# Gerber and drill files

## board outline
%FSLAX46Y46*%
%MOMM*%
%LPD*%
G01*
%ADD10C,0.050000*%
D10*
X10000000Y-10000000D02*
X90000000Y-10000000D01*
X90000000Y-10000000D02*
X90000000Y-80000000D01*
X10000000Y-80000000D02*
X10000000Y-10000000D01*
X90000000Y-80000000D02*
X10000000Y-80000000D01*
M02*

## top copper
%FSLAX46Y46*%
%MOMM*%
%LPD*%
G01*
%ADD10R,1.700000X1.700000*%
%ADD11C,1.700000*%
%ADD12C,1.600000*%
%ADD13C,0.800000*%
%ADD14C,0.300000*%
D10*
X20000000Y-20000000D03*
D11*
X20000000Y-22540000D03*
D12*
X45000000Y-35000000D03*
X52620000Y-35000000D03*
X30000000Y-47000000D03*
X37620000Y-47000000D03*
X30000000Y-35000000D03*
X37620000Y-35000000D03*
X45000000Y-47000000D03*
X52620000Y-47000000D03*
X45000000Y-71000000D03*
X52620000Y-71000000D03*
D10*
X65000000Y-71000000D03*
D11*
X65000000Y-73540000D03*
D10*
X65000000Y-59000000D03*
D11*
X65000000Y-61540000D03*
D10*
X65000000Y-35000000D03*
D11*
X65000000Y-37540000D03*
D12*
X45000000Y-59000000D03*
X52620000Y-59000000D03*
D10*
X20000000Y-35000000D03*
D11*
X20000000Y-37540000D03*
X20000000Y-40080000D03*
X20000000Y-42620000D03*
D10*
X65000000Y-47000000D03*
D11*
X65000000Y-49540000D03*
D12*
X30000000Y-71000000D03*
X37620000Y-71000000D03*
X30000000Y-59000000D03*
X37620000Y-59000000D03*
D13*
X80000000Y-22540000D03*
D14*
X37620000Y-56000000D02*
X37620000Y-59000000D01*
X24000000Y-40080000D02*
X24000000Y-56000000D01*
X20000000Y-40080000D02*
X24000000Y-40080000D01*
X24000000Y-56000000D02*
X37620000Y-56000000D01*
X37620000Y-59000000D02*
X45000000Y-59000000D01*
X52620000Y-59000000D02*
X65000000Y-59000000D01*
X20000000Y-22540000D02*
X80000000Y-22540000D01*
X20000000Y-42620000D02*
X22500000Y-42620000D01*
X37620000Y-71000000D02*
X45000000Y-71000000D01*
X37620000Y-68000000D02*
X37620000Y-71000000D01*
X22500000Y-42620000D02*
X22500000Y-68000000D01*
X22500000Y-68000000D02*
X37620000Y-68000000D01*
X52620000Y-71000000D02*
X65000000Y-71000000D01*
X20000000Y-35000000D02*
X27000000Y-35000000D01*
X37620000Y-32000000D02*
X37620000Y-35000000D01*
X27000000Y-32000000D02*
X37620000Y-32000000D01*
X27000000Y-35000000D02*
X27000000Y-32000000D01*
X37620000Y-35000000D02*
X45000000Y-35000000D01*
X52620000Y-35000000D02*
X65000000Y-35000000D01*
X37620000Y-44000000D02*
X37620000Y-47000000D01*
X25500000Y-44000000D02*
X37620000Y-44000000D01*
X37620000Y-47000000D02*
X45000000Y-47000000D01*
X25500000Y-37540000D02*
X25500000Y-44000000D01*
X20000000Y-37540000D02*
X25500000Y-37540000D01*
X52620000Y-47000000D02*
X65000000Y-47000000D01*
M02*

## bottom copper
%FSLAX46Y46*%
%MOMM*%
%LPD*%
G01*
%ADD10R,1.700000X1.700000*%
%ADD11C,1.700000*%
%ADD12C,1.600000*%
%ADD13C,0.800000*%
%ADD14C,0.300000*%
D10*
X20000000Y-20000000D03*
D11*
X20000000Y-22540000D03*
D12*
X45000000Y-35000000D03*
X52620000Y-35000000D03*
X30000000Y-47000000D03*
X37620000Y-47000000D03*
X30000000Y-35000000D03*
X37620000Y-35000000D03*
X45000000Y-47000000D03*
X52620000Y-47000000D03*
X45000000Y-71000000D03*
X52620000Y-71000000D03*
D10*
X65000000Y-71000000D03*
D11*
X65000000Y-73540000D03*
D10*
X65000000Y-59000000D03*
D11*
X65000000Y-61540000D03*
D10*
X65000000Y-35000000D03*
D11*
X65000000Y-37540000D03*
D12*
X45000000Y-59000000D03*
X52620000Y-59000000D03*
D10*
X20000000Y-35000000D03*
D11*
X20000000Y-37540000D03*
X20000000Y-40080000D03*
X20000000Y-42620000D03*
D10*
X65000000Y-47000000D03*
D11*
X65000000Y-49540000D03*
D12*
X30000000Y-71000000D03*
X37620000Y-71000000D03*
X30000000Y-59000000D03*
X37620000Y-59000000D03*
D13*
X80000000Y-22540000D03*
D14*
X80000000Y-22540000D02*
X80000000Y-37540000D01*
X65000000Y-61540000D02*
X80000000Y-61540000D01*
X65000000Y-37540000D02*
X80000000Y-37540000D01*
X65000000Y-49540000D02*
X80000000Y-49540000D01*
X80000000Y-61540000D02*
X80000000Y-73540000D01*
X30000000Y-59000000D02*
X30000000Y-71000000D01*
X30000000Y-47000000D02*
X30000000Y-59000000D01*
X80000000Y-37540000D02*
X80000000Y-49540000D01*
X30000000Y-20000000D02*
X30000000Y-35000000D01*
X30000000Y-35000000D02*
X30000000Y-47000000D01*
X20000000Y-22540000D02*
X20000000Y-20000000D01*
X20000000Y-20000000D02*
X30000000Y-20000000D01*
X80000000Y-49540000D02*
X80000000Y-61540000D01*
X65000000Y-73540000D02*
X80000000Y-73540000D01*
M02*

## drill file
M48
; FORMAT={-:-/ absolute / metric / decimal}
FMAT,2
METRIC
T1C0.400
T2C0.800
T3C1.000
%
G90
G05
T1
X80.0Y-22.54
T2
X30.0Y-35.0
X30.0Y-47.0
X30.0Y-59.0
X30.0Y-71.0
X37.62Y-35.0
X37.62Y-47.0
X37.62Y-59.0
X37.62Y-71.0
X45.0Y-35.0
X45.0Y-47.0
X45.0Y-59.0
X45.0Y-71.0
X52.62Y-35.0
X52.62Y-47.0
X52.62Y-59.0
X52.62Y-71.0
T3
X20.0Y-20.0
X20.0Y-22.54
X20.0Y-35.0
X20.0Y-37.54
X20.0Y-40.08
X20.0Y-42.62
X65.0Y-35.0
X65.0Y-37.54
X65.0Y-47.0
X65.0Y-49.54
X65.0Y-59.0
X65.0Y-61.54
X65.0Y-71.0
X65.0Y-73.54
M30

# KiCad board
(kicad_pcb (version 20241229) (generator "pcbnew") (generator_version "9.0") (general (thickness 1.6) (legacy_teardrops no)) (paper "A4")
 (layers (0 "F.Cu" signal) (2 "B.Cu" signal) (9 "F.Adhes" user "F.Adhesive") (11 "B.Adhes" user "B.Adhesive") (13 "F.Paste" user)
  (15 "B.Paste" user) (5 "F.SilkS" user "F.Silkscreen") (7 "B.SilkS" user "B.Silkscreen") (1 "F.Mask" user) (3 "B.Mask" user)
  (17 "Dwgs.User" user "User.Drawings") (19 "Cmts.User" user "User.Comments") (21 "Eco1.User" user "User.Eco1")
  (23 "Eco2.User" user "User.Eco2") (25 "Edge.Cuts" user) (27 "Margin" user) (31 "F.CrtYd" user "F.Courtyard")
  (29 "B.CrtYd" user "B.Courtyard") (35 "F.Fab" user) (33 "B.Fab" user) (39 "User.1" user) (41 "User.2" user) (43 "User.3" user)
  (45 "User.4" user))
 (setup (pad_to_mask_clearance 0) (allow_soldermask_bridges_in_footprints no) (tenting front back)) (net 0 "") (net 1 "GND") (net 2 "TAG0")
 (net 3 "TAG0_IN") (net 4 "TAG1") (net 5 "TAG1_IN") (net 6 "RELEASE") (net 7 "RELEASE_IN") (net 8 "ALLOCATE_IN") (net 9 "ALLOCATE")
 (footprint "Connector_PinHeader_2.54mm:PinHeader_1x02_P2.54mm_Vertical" (layer "F.Cu") (at 20 20)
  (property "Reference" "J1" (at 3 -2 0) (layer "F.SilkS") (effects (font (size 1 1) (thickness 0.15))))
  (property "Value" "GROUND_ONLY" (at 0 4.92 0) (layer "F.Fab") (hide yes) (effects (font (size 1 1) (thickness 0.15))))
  (pad "1" thru_hole rect (at 0 0) (size 1.7 1.7) (drill 1) (layers "*.Cu" "*.Mask") (remove_unused_layers no) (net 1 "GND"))
  (pad "2" thru_hole circle (at 0 2.54) (size 1.7 1.7) (drill 1) (layers "*.Cu" "*.Mask") (remove_unused_layers no) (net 1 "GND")))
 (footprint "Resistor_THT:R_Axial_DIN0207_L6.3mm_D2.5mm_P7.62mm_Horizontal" (layer "F.Cu") (at 45 35)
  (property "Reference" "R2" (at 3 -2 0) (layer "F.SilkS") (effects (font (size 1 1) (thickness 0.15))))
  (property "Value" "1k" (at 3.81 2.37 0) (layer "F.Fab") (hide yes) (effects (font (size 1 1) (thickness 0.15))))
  (pad "1" thru_hole circle (at 0 0) (size 1.6 1.6) (drill 0.8) (layers "*.Cu" "*.Mask") (remove_unused_layers no) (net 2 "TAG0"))
  (pad "2" thru_hole circle (at 7.62 0) (size 1.6 1.6) (drill 0.8) (layers "*.Cu" "*.Mask") (remove_unused_layers no) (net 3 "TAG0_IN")))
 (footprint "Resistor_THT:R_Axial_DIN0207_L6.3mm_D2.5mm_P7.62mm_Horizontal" (layer "F.Cu") (at 30 47)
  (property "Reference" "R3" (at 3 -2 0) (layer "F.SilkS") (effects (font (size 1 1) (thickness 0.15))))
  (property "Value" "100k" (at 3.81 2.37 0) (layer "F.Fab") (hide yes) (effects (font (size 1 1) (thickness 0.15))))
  (pad "1" thru_hole circle (at 0 0) (size 1.6 1.6) (drill 0.8) (layers "*.Cu" "*.Mask") (remove_unused_layers no) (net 1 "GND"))
  (pad "2" thru_hole circle (at 7.62 0) (size 1.6 1.6) (drill 0.8) (layers "*.Cu" "*.Mask") (remove_unused_layers no) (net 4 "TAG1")))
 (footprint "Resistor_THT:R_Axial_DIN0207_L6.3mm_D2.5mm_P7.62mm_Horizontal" (layer "F.Cu") (at 30 35)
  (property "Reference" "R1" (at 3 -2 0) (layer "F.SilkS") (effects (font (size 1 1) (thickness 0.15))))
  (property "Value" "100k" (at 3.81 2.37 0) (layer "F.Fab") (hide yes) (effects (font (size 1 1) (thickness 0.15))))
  (pad "1" thru_hole circle (at 0 0) (size 1.6 1.6) (drill 0.8) (layers "*.Cu" "*.Mask") (remove_unused_layers no) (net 1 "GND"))
  (pad "2" thru_hole circle (at 7.62 0) (size 1.6 1.6) (drill 0.8) (layers "*.Cu" "*.Mask") (remove_unused_layers no) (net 2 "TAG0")))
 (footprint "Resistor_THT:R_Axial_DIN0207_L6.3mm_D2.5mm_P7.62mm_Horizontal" (layer "F.Cu") (at 45 47)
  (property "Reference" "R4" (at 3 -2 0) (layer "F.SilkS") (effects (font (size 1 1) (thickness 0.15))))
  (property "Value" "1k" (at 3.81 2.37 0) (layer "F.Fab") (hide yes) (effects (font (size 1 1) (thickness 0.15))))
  (pad "1" thru_hole circle (at 0 0) (size 1.6 1.6) (drill 0.8) (layers "*.Cu" "*.Mask") (remove_unused_layers no) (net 4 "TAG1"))
  (pad "2" thru_hole circle (at 7.62 0) (size 1.6 1.6) (drill 0.8) (layers "*.Cu" "*.Mask") (remove_unused_layers no) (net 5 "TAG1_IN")))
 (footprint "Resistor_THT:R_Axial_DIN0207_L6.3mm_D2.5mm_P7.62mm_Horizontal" (layer "F.Cu") (at 45 71)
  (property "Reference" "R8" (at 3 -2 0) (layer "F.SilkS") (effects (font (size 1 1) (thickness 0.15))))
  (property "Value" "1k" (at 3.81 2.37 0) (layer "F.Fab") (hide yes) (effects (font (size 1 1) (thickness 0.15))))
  (pad "1" thru_hole circle (at 0 0) (size 1.6 1.6) (drill 0.8) (layers "*.Cu" "*.Mask") (remove_unused_layers no) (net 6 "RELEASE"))
  (pad "2" thru_hole circle (at 7.62 0) (size 1.6 1.6) (drill 0.8) (layers "*.Cu" "*.Mask") (remove_unused_layers no) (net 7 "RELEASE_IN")))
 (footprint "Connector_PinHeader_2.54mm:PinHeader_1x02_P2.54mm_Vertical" (layer "F.Cu") (at 65 71)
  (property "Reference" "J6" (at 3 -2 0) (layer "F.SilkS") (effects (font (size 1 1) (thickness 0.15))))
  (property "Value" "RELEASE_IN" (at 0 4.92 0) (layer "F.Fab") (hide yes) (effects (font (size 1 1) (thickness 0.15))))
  (pad "1" thru_hole rect (at 0 0) (size 1.7 1.7) (drill 1) (layers "*.Cu" "*.Mask") (remove_unused_layers no) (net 7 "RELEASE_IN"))
  (pad "2" thru_hole circle (at 0 2.54) (size 1.7 1.7) (drill 1) (layers "*.Cu" "*.Mask") (remove_unused_layers no) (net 1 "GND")))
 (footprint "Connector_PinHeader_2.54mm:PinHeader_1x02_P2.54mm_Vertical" (layer "F.Cu") (at 65 59)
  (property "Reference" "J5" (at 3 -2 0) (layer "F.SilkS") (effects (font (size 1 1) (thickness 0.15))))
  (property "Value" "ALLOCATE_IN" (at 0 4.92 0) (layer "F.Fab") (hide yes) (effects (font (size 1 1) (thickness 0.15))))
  (pad "1" thru_hole rect (at 0 0) (size 1.7 1.7) (drill 1) (layers "*.Cu" "*.Mask") (remove_unused_layers no) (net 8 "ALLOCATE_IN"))
  (pad "2" thru_hole circle (at 0 2.54) (size 1.7 1.7) (drill 1) (layers "*.Cu" "*.Mask") (remove_unused_layers no) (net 1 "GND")))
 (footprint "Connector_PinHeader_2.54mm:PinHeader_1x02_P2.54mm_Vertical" (layer "F.Cu") (at 65 35)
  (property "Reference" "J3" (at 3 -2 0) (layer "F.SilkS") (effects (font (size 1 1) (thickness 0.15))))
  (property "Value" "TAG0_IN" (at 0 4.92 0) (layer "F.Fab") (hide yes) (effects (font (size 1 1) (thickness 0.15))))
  (pad "1" thru_hole rect (at 0 0) (size 1.7 1.7) (drill 1) (layers "*.Cu" "*.Mask") (remove_unused_layers no) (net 3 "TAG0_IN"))
  (pad "2" thru_hole circle (at 0 2.54) (size 1.7 1.7) (drill 1) (layers "*.Cu" "*.Mask") (remove_unused_layers no) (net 1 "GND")))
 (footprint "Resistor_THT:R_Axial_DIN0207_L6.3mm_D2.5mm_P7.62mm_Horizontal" (layer "F.Cu") (at 45 59)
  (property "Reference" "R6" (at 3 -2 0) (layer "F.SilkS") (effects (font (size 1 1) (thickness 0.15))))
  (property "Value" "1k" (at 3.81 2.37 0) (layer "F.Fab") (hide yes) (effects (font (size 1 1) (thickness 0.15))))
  (pad "1" thru_hole circle (at 0 0) (size 1.6 1.6) (drill 0.8) (layers "*.Cu" "*.Mask") (remove_unused_layers no) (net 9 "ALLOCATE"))
  (pad "2" thru_hole circle (at 7.62 0) (size 1.6 1.6) (drill 0.8) (layers "*.Cu" "*.Mask") (remove_unused_layers no) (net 8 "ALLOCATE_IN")))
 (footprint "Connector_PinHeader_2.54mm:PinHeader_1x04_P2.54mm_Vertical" (layer "F.Cu") (at 20 35)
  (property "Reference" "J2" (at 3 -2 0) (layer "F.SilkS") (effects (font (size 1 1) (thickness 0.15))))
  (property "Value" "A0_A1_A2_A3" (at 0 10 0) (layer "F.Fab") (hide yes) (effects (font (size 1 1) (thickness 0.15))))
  (pad "1" thru_hole rect (at 0 0) (size 1.7 1.7) (drill 1) (layers "*.Cu" "*.Mask") (remove_unused_layers no) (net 2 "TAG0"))
  (pad "2" thru_hole circle (at 0 2.54) (size 1.7 1.7) (drill 1) (layers "*.Cu" "*.Mask") (remove_unused_layers no) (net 4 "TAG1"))
  (pad "3" thru_hole circle (at 0 5.08) (size 1.7 1.7) (drill 1) (layers "*.Cu" "*.Mask") (remove_unused_layers no) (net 9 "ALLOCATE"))
  (pad "4" thru_hole circle (at 0 7.62) (size 1.7 1.7) (drill 1) (layers "*.Cu" "*.Mask") (remove_unused_layers no) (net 6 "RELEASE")))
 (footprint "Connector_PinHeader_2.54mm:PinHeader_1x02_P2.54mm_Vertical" (layer "F.Cu") (at 65 47)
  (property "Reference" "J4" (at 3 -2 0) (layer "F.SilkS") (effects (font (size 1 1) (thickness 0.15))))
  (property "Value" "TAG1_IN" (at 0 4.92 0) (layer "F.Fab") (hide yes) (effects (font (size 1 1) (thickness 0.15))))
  (pad "1" thru_hole rect (at 0 0) (size 1.7 1.7) (drill 1) (layers "*.Cu" "*.Mask") (remove_unused_layers no) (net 5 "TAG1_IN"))
  (pad "2" thru_hole circle (at 0 2.54) (size 1.7 1.7) (drill 1) (layers "*.Cu" "*.Mask") (remove_unused_layers no) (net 1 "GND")))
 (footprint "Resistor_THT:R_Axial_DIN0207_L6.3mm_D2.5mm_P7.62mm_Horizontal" (layer "F.Cu") (at 30 71)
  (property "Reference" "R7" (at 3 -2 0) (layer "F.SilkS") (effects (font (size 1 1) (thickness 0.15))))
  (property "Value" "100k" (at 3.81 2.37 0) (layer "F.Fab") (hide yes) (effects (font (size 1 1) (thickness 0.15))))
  (pad "1" thru_hole circle (at 0 0) (size 1.6 1.6) (drill 0.8) (layers "*.Cu" "*.Mask") (remove_unused_layers no) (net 1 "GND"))
  (pad "2" thru_hole circle (at 7.62 0) (size 1.6 1.6) (drill 0.8) (layers "*.Cu" "*.Mask") (remove_unused_layers no) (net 6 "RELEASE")))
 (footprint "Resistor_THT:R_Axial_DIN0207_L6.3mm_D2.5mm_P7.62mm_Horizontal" (layer "F.Cu") (at 30 59)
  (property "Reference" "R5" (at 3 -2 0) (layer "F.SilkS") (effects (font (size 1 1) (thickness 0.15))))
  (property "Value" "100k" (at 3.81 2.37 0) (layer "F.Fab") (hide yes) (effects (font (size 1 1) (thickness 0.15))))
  (pad "1" thru_hole circle (at 0 0) (size 1.6 1.6) (drill 0.8) (layers "*.Cu" "*.Mask") (remove_unused_layers no) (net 1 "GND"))
  (pad "2" thru_hole circle (at 7.62 0) (size 1.6 1.6) (drill 0.8) (layers "*.Cu" "*.Mask") (remove_unused_layers no) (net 9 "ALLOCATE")))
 (gr_line (start 10 10) (end 90 10) (stroke (width 0.05) (type default)) (layer "Edge.Cuts"))
 (gr_line (start 90 10) (end 90 80) (stroke (width 0.05) (type default)) (layer "Edge.Cuts"))
 (gr_line (start 10 80) (end 10 10) (stroke (width 0.05) (type default)) (layer "Edge.Cuts"))
 (gr_line (start 90 80) (end 10 80) (stroke (width 0.05) (type default)) (layer "Edge.Cuts"))
 (segment (start 37.62 56) (end 37.62 59) (width 0.3) (layer "F.Cu") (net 9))
 (segment (start 24 40.08) (end 24 56) (width 0.3) (layer "F.Cu") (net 9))
 (segment (start 20 40.08) (end 24 40.08) (width 0.3) (layer "F.Cu") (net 9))
 (segment (start 24 56) (end 37.62 56) (width 0.3) (layer "F.Cu") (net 9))
 (segment (start 37.62 59) (end 45 59) (width 0.3) (layer "F.Cu") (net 9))
 (segment (start 52.62 59) (end 65 59) (width 0.3) (layer "F.Cu") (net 8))
 (segment (start 20 22.54) (end 80 22.54) (width 0.3) (layer "F.Cu") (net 1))
 (via (at 80 22.54) (size 0.8) (drill 0.4) (layers "F.Cu" "B.Cu") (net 1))
 (segment (start 80 22.54) (end 80 37.54) (width 0.3) (layer "B.Cu") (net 1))
 (segment (start 65 61.54) (end 80 61.54) (width 0.3) (layer "B.Cu") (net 1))
 (segment (start 65 37.54) (end 80 37.54) (width 0.3) (layer "B.Cu") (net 1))
 (segment (start 65 49.54) (end 80 49.54) (width 0.3) (layer "B.Cu") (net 1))
 (segment (start 80 61.54) (end 80 73.54) (width 0.3) (layer "B.Cu") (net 1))
 (segment (start 30 59) (end 30 71) (width 0.3) (layer "B.Cu") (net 1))
 (segment (start 30 47) (end 30 59) (width 0.3) (layer "B.Cu") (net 1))
 (segment (start 80 37.54) (end 80 49.54) (width 0.3) (layer "B.Cu") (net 1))
 (segment (start 30 20) (end 30 35) (width 0.3) (layer "B.Cu") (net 1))
 (segment (start 30 35) (end 30 47) (width 0.3) (layer "B.Cu") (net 1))
 (segment (start 20 22.54) (end 20 20) (width 0.3) (layer "B.Cu") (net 1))
 (segment (start 20 20) (end 30 20) (width 0.3) (layer "B.Cu") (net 1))
 (segment (start 80 49.54) (end 80 61.54) (width 0.3) (layer "B.Cu") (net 1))
 (segment (start 65 73.54) (end 80 73.54) (width 0.3) (layer "B.Cu") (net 1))
 (segment (start 20 42.62) (end 22.5 42.62) (width 0.3) (layer "F.Cu") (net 6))
 (segment (start 37.62 71) (end 45 71) (width 0.3) (layer "F.Cu") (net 6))
 (segment (start 37.62 68) (end 37.62 71) (width 0.3) (layer "F.Cu") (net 6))
 (segment (start 22.5 42.62) (end 22.5 68) (width 0.3) (layer "F.Cu") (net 6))
 (segment (start 22.5 68) (end 37.62 68) (width 0.3) (layer "F.Cu") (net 6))
 (segment (start 52.62 71) (end 65 71) (width 0.3) (layer "F.Cu") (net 7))
 (segment (start 20 35) (end 27 35) (width 0.3) (layer "F.Cu") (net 2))
 (segment (start 37.62 32) (end 37.62 35) (width 0.3) (layer "F.Cu") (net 2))
 (segment (start 27 32) (end 37.62 32) (width 0.3) (layer "F.Cu") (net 2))
 (segment (start 27 35) (end 27 32) (width 0.3) (layer "F.Cu") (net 2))
 (segment (start 37.62 35) (end 45 35) (width 0.3) (layer "F.Cu") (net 2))
 (segment (start 52.62 35) (end 65 35) (width 0.3) (layer "F.Cu") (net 3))
 (segment (start 37.62 44) (end 37.62 47) (width 0.3) (layer "F.Cu") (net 4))
 (segment (start 25.5 44) (end 37.62 44) (width 0.3) (layer "F.Cu") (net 4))
 (segment (start 37.62 47) (end 45 47) (width 0.3) (layer "F.Cu") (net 4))
 (segment (start 25.5 37.54) (end 25.5 44) (width 0.3) (layer "F.Cu") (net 4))
 (segment (start 20 37.54) (end 25.5 37.54) (width 0.3) (layer "F.Cu") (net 4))
 (segment (start 52.62 47) (end 65 47) (width 0.3) (layer "F.Cu") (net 5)))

